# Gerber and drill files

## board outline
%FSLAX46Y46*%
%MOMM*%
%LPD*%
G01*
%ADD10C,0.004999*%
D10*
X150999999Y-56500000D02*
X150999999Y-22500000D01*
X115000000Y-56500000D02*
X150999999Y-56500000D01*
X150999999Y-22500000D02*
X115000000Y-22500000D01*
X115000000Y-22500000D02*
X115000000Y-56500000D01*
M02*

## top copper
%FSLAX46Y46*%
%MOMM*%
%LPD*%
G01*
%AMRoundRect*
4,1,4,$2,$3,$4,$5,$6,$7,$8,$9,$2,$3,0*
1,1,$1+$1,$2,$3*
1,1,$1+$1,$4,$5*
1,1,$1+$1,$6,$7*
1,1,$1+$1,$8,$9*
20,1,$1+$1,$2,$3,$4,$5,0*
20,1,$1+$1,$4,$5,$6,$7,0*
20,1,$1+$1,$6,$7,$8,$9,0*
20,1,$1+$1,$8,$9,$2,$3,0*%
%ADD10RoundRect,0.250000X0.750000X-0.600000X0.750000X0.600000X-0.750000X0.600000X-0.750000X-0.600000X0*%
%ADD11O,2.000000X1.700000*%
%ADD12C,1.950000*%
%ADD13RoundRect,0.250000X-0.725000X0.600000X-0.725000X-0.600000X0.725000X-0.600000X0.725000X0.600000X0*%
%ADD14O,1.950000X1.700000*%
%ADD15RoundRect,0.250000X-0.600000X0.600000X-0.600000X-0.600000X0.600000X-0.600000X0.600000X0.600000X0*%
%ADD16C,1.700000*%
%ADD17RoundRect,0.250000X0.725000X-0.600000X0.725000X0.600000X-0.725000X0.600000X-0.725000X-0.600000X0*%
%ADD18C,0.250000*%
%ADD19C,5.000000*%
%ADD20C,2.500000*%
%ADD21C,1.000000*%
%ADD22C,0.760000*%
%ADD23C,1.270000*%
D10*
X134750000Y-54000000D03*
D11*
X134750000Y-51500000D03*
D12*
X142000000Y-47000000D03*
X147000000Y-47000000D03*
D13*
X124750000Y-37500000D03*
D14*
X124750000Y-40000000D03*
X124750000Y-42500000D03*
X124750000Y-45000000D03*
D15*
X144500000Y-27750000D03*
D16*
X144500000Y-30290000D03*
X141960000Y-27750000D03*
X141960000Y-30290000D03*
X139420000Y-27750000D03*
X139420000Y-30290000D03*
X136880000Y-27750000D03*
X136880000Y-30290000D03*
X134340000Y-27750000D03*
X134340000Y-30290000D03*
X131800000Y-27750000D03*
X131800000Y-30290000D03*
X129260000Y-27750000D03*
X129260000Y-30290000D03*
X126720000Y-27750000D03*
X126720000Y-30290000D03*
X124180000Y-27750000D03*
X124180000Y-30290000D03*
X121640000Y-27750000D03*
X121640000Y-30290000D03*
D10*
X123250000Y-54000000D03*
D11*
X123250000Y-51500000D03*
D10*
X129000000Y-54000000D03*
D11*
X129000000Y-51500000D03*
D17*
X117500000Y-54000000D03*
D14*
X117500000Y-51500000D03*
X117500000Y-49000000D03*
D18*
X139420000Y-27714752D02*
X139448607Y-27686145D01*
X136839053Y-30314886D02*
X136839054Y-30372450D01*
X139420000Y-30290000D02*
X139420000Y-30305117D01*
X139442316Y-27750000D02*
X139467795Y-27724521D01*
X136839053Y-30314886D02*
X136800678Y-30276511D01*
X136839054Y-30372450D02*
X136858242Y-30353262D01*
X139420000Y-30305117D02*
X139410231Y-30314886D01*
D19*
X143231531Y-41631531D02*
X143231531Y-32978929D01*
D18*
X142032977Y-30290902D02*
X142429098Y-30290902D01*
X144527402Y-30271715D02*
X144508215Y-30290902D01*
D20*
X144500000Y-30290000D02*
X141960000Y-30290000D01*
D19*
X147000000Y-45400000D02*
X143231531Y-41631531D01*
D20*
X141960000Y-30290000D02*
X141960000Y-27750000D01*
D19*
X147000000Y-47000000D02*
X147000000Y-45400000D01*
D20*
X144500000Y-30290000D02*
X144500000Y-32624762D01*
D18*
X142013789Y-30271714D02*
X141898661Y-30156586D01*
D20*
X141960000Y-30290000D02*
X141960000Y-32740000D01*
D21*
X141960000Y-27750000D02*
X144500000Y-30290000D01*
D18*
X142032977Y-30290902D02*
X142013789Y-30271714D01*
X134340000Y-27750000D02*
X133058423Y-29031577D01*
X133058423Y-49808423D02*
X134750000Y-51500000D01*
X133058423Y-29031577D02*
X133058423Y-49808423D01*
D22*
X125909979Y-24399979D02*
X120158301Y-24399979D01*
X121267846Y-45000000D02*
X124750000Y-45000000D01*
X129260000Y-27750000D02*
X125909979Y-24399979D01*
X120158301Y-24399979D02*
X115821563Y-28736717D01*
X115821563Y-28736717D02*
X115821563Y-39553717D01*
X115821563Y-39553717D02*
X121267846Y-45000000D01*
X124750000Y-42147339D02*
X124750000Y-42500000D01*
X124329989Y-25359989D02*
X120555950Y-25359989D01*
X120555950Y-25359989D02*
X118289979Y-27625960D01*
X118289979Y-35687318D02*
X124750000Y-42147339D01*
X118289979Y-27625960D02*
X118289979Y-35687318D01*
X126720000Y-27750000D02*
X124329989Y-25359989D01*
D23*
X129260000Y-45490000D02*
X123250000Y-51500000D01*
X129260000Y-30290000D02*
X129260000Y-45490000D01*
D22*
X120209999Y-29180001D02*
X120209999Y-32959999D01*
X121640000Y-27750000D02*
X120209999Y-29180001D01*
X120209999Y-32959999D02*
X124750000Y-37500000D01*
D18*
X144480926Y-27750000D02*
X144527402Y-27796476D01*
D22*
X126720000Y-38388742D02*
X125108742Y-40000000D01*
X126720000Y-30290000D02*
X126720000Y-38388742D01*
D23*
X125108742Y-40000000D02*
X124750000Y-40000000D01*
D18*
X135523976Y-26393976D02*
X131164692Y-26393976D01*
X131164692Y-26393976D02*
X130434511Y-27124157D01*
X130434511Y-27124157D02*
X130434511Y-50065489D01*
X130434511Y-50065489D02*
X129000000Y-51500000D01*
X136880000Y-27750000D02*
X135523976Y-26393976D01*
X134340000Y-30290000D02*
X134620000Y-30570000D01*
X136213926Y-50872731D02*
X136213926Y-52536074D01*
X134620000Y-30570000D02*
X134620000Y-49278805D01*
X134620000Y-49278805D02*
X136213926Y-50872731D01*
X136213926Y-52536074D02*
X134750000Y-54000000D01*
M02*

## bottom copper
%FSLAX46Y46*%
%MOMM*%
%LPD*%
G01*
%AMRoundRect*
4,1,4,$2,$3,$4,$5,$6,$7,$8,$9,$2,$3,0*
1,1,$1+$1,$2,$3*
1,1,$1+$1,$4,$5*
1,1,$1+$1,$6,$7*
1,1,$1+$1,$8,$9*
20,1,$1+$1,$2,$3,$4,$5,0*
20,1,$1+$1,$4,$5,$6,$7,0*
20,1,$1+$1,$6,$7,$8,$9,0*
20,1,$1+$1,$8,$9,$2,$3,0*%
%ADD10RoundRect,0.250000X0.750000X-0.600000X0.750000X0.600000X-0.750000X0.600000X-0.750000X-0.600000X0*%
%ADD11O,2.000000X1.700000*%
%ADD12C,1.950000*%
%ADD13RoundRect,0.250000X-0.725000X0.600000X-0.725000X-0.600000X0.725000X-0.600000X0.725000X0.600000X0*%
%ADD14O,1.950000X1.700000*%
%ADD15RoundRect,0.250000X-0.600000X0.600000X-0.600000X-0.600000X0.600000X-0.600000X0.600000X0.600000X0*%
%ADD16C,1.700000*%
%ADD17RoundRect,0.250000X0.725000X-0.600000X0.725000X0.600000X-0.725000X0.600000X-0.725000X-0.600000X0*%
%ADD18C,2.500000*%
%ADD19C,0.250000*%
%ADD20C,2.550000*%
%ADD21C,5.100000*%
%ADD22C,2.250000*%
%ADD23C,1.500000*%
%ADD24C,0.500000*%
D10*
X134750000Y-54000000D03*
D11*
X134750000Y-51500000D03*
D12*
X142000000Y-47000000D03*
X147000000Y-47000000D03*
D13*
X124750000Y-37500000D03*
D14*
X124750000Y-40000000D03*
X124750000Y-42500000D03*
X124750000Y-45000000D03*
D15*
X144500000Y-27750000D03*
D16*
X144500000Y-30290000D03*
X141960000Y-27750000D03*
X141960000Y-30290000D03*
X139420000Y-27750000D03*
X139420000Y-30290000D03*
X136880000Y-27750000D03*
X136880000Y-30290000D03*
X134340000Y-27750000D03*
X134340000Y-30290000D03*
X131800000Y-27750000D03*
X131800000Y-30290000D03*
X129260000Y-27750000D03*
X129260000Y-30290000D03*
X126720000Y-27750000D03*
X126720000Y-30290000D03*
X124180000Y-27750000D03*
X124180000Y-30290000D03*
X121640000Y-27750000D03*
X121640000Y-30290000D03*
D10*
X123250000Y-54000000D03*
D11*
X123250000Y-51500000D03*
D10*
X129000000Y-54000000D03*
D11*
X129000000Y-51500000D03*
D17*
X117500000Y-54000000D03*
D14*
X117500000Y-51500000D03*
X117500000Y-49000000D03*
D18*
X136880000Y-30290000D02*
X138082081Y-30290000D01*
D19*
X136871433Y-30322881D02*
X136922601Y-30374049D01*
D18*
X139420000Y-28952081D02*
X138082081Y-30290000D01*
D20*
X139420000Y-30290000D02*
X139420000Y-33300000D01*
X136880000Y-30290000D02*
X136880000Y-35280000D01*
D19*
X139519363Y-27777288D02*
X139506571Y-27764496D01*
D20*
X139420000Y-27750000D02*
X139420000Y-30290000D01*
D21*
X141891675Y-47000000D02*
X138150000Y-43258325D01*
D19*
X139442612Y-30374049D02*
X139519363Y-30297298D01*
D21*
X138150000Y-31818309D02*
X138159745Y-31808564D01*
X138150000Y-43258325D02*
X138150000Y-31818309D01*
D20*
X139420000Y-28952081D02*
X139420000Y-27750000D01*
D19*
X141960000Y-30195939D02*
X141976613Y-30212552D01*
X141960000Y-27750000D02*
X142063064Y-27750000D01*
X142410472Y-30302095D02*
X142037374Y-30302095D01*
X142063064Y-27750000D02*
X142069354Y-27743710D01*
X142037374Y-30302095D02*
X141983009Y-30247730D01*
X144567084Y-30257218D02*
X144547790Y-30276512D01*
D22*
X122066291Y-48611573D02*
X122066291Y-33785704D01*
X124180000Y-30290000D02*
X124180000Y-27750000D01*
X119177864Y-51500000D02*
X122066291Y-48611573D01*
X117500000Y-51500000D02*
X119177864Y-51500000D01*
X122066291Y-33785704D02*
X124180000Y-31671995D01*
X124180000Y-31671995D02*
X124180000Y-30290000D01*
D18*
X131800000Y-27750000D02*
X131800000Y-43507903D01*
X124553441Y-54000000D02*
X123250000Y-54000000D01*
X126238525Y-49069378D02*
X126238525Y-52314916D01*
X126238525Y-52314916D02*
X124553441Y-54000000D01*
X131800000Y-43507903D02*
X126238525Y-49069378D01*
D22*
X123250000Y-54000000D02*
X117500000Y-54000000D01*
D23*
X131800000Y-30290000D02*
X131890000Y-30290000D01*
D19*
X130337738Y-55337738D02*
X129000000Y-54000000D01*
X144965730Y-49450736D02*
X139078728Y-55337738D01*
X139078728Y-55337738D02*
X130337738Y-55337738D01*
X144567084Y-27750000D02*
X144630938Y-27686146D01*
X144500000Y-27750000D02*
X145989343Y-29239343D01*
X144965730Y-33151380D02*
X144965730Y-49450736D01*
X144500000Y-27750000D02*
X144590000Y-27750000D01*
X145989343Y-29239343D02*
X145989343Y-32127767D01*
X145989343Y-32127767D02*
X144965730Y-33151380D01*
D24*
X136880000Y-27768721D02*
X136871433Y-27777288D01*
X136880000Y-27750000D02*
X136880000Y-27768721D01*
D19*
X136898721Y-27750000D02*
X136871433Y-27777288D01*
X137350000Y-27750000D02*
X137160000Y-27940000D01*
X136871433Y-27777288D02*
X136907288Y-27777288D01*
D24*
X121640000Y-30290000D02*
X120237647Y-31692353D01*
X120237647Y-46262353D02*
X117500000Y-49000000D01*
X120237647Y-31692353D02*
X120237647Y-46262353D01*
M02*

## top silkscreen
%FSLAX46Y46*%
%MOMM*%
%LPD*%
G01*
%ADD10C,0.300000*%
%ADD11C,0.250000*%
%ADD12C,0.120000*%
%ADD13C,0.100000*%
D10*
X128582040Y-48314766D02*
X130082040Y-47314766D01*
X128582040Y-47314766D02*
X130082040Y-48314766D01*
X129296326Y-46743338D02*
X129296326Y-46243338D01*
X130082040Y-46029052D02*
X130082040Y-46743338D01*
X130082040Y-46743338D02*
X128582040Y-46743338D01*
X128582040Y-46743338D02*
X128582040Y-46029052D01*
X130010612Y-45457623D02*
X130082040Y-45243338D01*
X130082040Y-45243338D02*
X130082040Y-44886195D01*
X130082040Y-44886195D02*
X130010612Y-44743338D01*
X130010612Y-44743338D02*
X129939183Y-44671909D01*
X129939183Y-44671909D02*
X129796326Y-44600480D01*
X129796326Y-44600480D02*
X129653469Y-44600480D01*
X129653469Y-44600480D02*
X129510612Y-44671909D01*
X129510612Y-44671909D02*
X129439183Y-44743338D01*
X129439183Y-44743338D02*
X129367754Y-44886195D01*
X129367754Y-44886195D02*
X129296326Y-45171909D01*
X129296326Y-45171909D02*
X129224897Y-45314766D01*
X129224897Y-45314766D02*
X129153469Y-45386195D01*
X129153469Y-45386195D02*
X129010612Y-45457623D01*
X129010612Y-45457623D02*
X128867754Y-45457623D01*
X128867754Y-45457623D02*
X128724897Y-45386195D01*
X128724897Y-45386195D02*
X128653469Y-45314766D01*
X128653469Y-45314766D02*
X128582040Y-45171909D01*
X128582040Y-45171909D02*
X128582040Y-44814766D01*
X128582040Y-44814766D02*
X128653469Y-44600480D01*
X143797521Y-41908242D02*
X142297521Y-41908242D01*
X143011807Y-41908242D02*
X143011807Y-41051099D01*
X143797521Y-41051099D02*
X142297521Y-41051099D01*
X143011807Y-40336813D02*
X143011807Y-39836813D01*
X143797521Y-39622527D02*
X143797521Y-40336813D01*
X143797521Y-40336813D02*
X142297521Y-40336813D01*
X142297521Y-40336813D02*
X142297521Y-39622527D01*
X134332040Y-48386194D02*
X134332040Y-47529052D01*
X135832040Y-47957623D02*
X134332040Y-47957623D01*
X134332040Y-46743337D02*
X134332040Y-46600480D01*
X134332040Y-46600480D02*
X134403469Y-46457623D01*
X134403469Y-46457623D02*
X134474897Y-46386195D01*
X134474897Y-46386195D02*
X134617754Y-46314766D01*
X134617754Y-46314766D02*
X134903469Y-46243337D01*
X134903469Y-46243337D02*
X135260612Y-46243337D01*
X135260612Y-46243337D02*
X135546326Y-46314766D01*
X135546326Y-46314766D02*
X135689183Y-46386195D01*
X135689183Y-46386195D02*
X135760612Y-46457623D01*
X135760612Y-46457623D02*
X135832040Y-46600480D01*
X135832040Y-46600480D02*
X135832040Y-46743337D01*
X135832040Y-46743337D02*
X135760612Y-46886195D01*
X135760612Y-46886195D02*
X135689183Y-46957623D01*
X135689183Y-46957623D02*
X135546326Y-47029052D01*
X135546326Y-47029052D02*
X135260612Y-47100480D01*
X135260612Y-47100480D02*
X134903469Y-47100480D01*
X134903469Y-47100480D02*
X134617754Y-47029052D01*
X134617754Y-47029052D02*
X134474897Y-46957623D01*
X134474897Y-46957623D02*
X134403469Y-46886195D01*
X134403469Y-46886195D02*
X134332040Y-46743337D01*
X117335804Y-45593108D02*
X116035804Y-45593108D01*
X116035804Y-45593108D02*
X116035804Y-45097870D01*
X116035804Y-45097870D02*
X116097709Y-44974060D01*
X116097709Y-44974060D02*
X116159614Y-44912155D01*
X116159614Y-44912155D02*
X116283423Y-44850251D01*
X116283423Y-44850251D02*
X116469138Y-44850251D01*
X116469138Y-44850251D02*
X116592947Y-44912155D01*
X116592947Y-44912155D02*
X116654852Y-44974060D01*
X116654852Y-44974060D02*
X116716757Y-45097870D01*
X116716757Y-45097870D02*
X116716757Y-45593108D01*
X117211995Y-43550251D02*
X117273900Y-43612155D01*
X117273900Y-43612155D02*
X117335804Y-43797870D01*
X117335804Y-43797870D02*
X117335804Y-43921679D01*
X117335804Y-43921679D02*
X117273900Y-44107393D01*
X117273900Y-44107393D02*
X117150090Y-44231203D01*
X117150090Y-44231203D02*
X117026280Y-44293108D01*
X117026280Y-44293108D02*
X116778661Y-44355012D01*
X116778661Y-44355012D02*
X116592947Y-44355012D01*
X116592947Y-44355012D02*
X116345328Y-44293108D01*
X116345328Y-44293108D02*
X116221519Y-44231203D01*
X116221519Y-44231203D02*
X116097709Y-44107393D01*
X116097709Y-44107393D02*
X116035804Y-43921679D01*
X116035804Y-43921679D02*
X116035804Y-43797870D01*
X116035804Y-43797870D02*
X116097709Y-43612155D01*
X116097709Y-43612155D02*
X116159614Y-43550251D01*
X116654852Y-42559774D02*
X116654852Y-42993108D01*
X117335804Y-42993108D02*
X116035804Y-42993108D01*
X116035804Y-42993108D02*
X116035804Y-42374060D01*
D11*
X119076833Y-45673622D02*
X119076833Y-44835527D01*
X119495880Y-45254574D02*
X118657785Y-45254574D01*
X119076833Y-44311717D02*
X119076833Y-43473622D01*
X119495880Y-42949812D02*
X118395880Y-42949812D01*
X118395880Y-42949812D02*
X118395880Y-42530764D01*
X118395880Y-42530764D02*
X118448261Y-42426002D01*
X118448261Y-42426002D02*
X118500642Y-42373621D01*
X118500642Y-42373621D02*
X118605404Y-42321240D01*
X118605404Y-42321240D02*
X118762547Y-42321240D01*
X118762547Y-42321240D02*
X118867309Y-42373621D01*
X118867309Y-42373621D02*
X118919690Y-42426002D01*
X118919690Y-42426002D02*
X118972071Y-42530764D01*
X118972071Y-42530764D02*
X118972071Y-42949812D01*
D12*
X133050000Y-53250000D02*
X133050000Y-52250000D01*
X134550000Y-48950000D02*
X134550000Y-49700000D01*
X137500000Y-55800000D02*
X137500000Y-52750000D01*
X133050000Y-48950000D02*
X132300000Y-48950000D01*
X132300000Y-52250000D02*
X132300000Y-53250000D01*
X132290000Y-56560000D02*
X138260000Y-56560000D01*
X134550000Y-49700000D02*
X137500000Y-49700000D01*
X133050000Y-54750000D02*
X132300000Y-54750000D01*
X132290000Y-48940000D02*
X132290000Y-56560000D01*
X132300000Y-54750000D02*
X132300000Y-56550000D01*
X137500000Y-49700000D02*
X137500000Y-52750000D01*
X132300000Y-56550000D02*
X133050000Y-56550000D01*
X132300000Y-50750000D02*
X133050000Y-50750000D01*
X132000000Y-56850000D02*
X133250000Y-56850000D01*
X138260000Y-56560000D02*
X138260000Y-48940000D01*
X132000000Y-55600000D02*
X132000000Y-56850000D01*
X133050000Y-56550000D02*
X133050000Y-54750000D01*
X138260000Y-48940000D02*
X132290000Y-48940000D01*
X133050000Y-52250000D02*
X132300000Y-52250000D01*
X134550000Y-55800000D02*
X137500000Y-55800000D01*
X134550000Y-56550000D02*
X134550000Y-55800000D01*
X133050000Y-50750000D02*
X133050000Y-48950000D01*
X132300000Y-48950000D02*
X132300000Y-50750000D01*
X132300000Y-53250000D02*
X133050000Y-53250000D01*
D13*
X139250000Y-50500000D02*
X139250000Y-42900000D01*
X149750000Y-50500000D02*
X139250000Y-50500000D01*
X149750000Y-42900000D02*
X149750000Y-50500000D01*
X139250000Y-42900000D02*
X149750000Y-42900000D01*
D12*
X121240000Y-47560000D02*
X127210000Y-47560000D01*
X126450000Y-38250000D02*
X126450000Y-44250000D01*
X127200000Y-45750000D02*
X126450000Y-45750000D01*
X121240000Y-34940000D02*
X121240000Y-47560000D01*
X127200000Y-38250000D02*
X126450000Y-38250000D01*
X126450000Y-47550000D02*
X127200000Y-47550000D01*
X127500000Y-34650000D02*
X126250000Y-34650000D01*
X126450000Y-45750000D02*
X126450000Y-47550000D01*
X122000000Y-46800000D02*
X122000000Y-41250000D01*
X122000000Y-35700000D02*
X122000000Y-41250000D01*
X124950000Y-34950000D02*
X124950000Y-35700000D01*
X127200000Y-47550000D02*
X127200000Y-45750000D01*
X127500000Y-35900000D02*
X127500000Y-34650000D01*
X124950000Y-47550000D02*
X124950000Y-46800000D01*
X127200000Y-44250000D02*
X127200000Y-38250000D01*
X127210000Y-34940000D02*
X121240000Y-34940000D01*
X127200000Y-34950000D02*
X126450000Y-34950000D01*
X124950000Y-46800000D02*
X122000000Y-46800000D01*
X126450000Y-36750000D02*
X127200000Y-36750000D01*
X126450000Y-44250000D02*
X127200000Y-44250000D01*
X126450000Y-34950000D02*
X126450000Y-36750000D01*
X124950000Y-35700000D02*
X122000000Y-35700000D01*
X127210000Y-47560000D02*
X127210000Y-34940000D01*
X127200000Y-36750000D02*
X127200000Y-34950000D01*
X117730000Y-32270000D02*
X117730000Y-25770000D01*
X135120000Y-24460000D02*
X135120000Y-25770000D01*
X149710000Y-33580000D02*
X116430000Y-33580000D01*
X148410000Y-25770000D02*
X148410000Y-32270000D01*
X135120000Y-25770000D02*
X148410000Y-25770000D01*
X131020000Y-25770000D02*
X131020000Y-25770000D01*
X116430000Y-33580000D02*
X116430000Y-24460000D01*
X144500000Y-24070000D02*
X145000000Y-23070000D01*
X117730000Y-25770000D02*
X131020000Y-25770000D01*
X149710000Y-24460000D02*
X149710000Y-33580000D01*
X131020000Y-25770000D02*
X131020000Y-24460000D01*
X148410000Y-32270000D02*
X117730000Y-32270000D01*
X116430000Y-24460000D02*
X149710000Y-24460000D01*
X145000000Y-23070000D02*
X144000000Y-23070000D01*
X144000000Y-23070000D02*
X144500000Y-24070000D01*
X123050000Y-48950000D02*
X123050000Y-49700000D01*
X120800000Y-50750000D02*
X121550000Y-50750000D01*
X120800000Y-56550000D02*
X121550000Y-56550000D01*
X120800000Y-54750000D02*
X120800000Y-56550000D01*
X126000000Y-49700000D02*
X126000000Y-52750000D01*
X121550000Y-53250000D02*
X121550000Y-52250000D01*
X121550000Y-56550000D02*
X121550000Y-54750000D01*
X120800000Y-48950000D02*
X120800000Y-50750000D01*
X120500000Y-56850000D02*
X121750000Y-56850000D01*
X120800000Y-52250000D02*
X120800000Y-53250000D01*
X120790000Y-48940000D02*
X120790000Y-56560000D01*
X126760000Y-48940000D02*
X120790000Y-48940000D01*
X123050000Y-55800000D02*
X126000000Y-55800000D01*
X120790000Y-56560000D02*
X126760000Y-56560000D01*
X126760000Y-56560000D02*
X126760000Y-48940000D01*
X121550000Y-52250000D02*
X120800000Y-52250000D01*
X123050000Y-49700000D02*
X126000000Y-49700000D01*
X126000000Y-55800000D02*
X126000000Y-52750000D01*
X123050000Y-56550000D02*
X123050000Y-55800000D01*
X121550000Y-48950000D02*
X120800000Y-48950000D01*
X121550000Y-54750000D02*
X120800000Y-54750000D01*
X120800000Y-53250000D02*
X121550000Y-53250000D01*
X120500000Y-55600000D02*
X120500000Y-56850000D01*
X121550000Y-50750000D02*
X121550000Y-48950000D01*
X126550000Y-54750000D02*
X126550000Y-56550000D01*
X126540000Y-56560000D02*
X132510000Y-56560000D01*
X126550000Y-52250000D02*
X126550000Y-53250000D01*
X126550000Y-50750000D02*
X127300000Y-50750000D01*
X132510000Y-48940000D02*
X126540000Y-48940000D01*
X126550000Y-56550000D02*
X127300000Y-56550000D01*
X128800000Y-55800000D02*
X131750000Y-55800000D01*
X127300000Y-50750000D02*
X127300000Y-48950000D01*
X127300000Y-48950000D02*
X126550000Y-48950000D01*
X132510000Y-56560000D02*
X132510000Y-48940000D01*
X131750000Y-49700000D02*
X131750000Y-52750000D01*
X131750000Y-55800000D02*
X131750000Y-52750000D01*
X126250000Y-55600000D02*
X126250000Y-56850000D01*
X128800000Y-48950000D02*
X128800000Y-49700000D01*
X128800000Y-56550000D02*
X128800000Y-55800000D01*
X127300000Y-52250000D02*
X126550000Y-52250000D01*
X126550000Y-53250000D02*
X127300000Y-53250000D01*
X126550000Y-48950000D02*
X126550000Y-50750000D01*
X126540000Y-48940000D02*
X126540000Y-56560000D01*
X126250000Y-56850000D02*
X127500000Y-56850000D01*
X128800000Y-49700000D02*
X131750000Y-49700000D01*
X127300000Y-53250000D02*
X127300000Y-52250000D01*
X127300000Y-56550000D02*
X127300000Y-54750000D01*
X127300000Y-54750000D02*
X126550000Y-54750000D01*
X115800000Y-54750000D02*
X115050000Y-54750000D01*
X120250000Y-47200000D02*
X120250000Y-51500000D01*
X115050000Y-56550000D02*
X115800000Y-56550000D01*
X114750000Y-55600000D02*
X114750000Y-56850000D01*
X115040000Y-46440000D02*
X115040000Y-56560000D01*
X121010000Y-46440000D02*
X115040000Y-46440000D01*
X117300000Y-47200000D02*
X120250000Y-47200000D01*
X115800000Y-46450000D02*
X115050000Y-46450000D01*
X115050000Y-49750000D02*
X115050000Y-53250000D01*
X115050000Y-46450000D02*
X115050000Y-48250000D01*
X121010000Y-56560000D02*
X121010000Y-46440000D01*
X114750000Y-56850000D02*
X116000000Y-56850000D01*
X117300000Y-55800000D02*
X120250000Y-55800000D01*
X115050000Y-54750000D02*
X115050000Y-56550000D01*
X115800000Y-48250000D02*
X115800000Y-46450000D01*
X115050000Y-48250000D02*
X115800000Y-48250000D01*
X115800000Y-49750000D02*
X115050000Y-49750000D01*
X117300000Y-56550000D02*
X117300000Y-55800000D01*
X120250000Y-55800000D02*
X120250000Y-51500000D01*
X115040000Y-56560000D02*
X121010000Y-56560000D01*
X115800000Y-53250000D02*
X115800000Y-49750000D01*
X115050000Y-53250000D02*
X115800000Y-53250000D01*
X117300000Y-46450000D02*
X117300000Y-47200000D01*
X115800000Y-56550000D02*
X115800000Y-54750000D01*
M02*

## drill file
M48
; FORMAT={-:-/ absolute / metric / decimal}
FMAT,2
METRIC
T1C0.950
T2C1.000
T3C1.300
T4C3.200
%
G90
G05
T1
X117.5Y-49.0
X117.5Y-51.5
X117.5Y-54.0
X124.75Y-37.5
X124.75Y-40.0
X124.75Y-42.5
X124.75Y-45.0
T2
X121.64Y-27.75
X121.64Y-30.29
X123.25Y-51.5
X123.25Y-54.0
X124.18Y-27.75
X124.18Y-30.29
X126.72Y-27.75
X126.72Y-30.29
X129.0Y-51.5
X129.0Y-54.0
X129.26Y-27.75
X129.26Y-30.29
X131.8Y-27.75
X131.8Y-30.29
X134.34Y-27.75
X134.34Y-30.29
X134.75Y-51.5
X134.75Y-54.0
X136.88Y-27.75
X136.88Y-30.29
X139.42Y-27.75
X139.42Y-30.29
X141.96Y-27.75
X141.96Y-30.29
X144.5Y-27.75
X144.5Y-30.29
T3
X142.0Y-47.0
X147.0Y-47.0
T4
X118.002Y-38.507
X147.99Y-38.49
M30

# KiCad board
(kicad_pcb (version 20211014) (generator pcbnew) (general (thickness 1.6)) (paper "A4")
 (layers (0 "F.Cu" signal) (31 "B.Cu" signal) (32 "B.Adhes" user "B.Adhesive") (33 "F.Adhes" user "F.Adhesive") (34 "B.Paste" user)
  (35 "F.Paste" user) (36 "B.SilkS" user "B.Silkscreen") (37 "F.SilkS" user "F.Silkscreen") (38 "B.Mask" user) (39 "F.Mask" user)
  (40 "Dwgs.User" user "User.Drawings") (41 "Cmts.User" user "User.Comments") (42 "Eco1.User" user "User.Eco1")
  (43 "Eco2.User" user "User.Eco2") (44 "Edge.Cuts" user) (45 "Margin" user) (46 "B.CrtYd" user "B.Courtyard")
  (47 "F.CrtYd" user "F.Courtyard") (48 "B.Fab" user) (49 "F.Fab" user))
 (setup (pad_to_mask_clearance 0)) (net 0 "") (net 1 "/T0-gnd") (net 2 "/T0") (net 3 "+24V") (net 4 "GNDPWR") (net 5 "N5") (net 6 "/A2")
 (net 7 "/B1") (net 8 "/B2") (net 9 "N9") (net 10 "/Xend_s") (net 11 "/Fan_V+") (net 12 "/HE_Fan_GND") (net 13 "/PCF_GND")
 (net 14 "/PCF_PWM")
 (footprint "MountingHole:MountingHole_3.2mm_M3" (layer "F.Cu") (at 118.001564 38.507316)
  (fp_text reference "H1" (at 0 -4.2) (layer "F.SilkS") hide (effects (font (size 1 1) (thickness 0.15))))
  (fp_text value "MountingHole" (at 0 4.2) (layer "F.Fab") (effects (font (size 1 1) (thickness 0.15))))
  (pad "" np_thru_hole circle locked (at 0 0) (size 3.2 3.2) (drill 3.2) (layers *.Cu *.Mask)))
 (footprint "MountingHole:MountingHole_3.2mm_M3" (layer "F.Cu") (at 147.990137 38.490139)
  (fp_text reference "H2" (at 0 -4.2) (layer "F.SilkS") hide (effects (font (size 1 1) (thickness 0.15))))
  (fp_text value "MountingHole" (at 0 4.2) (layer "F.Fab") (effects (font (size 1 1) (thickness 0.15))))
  (pad "" np_thru_hole circle locked (at 0 0) (size 3.2 3.2) (drill 3.2) (layers *.Cu *.Mask)))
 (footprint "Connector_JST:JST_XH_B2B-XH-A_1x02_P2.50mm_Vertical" (layer "F.Cu") (at 134.75 54 90)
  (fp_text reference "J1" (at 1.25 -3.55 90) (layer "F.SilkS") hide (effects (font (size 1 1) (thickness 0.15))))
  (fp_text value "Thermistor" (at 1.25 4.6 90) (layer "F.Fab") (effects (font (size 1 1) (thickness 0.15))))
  (fp_line (start 0.75 -1.7) (end 1.75 -1.7) (layer "F.SilkS") (width 0.12))
  (fp_line (start 5.05 -0.2) (end 4.3 -0.2) (layer "F.SilkS") (width 0.12))
  (fp_line (start -1.8 2.75) (end 1.25 2.75) (layer "F.SilkS") (width 0.12))
  (fp_line (start 5.05 -1.7) (end 5.05 -2.45) (layer "F.SilkS") (width 0.12))
  (fp_line (start 1.75 -2.45) (end 0.75 -2.45) (layer "F.SilkS") (width 0.12))
  (fp_line (start -2.56 -2.46) (end -2.56 3.51) (layer "F.SilkS") (width 0.12))
  (fp_line (start 4.3 -0.2) (end 4.3 2.75) (layer "F.SilkS") (width 0.12))
  (fp_line (start -0.75 -1.7) (end -0.75 -2.45) (layer "F.SilkS") (width 0.12))
  (fp_line (start 5.06 -2.46) (end -2.56 -2.46) (layer "F.SilkS") (width 0.12))
  (fp_line (start -0.75 -2.45) (end -2.55 -2.45) (layer "F.SilkS") (width 0.12))
  (fp_line (start 4.3 2.75) (end 1.25 2.75) (layer "F.SilkS") (width 0.12))
  (fp_line (start -2.55 -2.45) (end -2.55 -1.7) (layer "F.SilkS") (width 0.12))
  (fp_line (start 3.25 -2.45) (end 3.25 -1.7) (layer "F.SilkS") (width 0.12))
  (fp_line (start -2.85 -2.75) (end -2.85 -1.5) (layer "F.SilkS") (width 0.12))
  (fp_line (start -2.56 3.51) (end 5.06 3.51) (layer "F.SilkS") (width 0.12))
  (fp_line (start -1.6 -2.75) (end -2.85 -2.75) (layer "F.SilkS") (width 0.12))
  (fp_line (start -2.55 -1.7) (end -0.75 -1.7) (layer "F.SilkS") (width 0.12))
  (fp_line (start 5.06 3.51) (end 5.06 -2.46) (layer "F.SilkS") (width 0.12))
  (fp_line (start 1.75 -1.7) (end 1.75 -2.45) (layer "F.SilkS") (width 0.12))
  (fp_line (start -1.8 -0.2) (end -1.8 2.75) (layer "F.SilkS") (width 0.12))
  (fp_line (start -2.55 -0.2) (end -1.8 -0.2) (layer "F.SilkS") (width 0.12))
  (fp_line (start 3.25 -1.7) (end 5.05 -1.7) (layer "F.SilkS") (width 0.12))
  (fp_line (start 5.05 -2.45) (end 3.25 -2.45) (layer "F.SilkS") (width 0.12))
  (fp_line (start 0.75 -2.45) (end 0.75 -1.7) (layer "F.SilkS") (width 0.12))
  (pad "1" thru_hole roundrect locked (at 0 0 90) (size 1.7 2) (drill 1) (layers *.Cu *.Mask) (roundrect_rratio 0.1470588235)
   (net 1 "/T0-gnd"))
  (pad "2" thru_hole oval locked (at 2.5 0 90) (size 1.7 2) (drill 1) (layers *.Cu *.Mask) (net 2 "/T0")))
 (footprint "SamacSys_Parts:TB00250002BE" (layer "F.Cu") (at 142 47)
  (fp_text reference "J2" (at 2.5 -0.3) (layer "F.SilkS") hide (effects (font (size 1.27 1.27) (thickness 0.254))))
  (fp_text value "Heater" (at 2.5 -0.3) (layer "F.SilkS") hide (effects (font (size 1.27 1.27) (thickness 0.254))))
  (fp_line (start -2.75 3.5) (end -2.75 -4.1) (layer "F.SilkS") (width 0.1))
  (fp_line (start 7.75 3.5) (end -2.75 3.5) (layer "F.SilkS") (width 0.1))
  (fp_line (start 7.75 -4.1) (end 7.75 3.5) (layer "F.SilkS") (width 0.1))
  (fp_line (start -2.75 -4.1) (end 7.75 -4.1) (layer "F.SilkS") (width 0.1))
  (pad "1" thru_hole circle locked (at 0 0) (size 1.95 1.95) (drill 1.3) (layers *.Cu *.Mask) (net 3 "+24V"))
  (pad "2" thru_hole circle locked (at 5 0) (size 1.95 1.95) (drill 1.3) (layers *.Cu *.Mask) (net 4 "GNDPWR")))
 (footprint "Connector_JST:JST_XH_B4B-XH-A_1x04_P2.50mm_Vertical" (layer "F.Cu") (at 124.75 37.5 -90)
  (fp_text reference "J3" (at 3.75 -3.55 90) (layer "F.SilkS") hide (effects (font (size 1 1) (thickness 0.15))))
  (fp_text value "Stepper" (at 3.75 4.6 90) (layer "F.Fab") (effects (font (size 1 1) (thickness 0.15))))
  (fp_line (start 10.06 3.51) (end 10.06 -2.46) (layer "F.SilkS") (width 0.12))
  (fp_line (start 0.75 -1.7) (end 6.75 -1.7) (layer "F.SilkS") (width 0.12))
  (fp_line (start 8.25 -2.45) (end 8.25 -1.7) (layer "F.SilkS") (width 0.12))
  (fp_line (start -2.56 3.51) (end 10.06 3.51) (layer "F.SilkS") (width 0.12))
  (fp_line (start 0.75 -2.45) (end 0.75 -1.7) (layer "F.SilkS") (width 0.12))
  (fp_line (start 10.05 -1.7) (end 10.05 -2.45) (layer "F.SilkS") (width 0.12))
  (fp_line (start -2.85 -2.75) (end -2.85 -1.5) (layer "F.SilkS") (width 0.12))
  (fp_line (start 8.25 -1.7) (end 10.05 -1.7) (layer "F.SilkS") (width 0.12))
  (fp_line (start 9.3 2.75) (end 3.75 2.75) (layer "F.SilkS") (width 0.12))
  (fp_line (start -1.8 2.75) (end 3.75 2.75) (layer "F.SilkS") (width 0.12))
  (fp_line (start -2.55 -0.2) (end -1.8 -0.2) (layer "F.SilkS") (width 0.12))
  (fp_line (start 10.05 -2.45) (end 8.25 -2.45) (layer "F.SilkS") (width 0.12))
  (fp_line (start -1.6 -2.75) (end -2.85 -2.75) (layer "F.SilkS") (width 0.12))
  (fp_line (start 10.05 -0.2) (end 9.3 -0.2) (layer "F.SilkS") (width 0.12))
  (fp_line (start 6.75 -2.45) (end 0.75 -2.45) (layer "F.SilkS") (width 0.12))
  (fp_line (start -2.56 -2.46) (end -2.56 3.51) (layer "F.SilkS") (width 0.12))
  (fp_line (start -2.55 -2.45) (end -2.55 -1.7) (layer "F.SilkS") (width 0.12))
  (fp_line (start 9.3 -0.2) (end 9.3 2.75) (layer "F.SilkS") (width 0.12))
  (fp_line (start -0.75 -1.7) (end -0.75 -2.45) (layer "F.SilkS") (width 0.12))
  (fp_line (start 6.75 -1.7) (end 6.75 -2.45) (layer "F.SilkS") (width 0.12))
  (fp_line (start -2.55 -1.7) (end -0.75 -1.7) (layer "F.SilkS") (width 0.12))
  (fp_line (start -1.8 -0.2) (end -1.8 2.75) (layer "F.SilkS") (width 0.12))
  (fp_line (start 10.06 -2.46) (end -2.56 -2.46) (layer "F.SilkS") (width 0.12))
  (fp_line (start -0.75 -2.45) (end -2.55 -2.45) (layer "F.SilkS") (width 0.12))
  (pad "1" thru_hole roundrect locked (at 0 0 270) (size 1.7 1.95) (drill 0.95) (layers *.Cu *.Mask) (roundrect_rratio 0.1470588235)
   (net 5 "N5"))
  (pad "2" thru_hole oval locked (at 2.5 0 270) (size 1.7 1.95) (drill 0.95) (layers *.Cu *.Mask) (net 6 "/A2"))
  (pad "3" thru_hole oval locked (at 5 0 270) (size 1.7 1.95) (drill 0.95) (layers *.Cu *.Mask) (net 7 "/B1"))
  (pad "4" thru_hole oval locked (at 7.5 0 270) (size 1.7 1.95) (drill 0.95) (layers *.Cu *.Mask) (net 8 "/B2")))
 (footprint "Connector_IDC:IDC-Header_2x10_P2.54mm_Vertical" (layer "F.Cu") (at 144.5 27.75 -90)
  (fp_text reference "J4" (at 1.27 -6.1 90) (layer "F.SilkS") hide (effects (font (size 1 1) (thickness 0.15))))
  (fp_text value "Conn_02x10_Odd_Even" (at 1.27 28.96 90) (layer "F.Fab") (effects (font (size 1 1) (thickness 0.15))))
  (fp_line (start 4.52 26.77) (end -1.98 26.77) (layer "F.SilkS") (width 0.12))
  (fp_line (start -3.29 9.38) (end -1.98 9.38) (layer "F.SilkS") (width 0.12))
  (fp_line (start 5.83 -5.21) (end 5.83 28.07) (layer "F.SilkS") (width 0.12))
  (fp_line (start -1.98 -3.91) (end 4.52 -3.91) (layer "F.SilkS") (width 0.12))
  (fp_line (start -1.98 9.38) (end -1.98 -3.91) (layer "F.SilkS") (width 0.12))
  (fp_line (start -1.98 13.48) (end -1.98 13.48) (layer "F.SilkS") (width 0.12))
  (fp_line (start 5.83 28.07) (end -3.29 28.07) (layer "F.SilkS") (width 0.12))
  (fp_line (start -3.68 0) (end -4.68 -0.5) (layer "F.SilkS") (width 0.12))
  (fp_line (start -1.98 26.77) (end -1.98 13.48) (layer "F.SilkS") (width 0.12))
  (fp_line (start -3.29 -5.21) (end 5.83 -5.21) (layer "F.SilkS") (width 0.12))
  (fp_line (start -1.98 13.48) (end -3.29 13.48) (layer "F.SilkS") (width 0.12))
  (fp_line (start 4.52 -3.91) (end 4.52 26.77) (layer "F.SilkS") (width 0.12))
  (fp_line (start -3.29 28.07) (end -3.29 -5.21) (layer "F.SilkS") (width 0.12))
  (fp_line (start -4.68 -0.5) (end -4.68 0.5) (layer "F.SilkS") (width 0.12))
  (fp_line (start -4.68 0.5) (end -3.68 0) (layer "F.SilkS") (width 0.12))
  (pad "1" thru_hole roundrect locked (at 0 0 270) (size 1.7 1.7) (drill 1) (layers *.Cu *.Mask) (roundrect_rratio 0.1470588235)
   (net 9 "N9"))
  (pad "2" thru_hole circle locked (at 2.54 0 270) (size 1.7 1.7) (drill 1) (layers *.Cu *.Mask) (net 4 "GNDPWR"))
  (pad "3" thru_hole circle locked (at 0 2.54 270) (size 1.7 1.7) (drill 1) (layers *.Cu *.Mask) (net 4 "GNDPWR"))
  (pad "4" thru_hole circle locked (at 2.54 2.54 270) (size 1.7 1.7) (drill 1) (layers *.Cu *.Mask) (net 4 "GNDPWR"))
  (pad "5" thru_hole circle locked (at 0 5.08 270) (size 1.7 1.7) (drill 1) (layers *.Cu *.Mask) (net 3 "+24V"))
  (pad "6" thru_hole circle locked (at 2.54 5.08 270) (size 1.7 1.7) (drill 1) (layers *.Cu *.Mask) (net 3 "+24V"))
  (pad "7" thru_hole circle locked (at 0 7.62 270) (size 1.7 1.7) (drill 1) (layers *.Cu *.Mask) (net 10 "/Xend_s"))
  (pad "8" thru_hole circle locked (at 2.54 7.62 270) (size 1.7 1.7) (drill 1) (layers *.Cu *.Mask) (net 3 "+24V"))
  (pad "9" thru_hole circle locked (at 0 10.16 270) (size 1.7 1.7) (drill 1) (layers *.Cu *.Mask) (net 2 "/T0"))
  (pad "10" thru_hole circle locked (at 2.54 10.16 270) (size 1.7 1.7) (drill 1) (layers *.Cu *.Mask) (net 1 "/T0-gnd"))
  (pad "11" thru_hole circle locked (at 0 12.7 270) (size 1.7 1.7) (drill 1) (layers *.Cu *.Mask) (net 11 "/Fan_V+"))
  (pad "12" thru_hole circle locked (at 2.54 12.7 270) (size 1.7 1.7) (drill 1) (layers *.Cu *.Mask) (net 11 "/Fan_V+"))
  (pad "13" thru_hole circle locked (at 0 15.24 270) (size 1.7 1.7) (drill 1) (layers *.Cu *.Mask) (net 8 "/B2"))
  (pad "14" thru_hole circle locked (at 2.54 15.24 270) (size 1.7 1.7) (drill 1) (layers *.Cu *.Mask) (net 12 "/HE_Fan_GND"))
  (pad "15" thru_hole circle locked (at 0 17.78 270) (size 1.7 1.7) (drill 1) (layers *.Cu *.Mask) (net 7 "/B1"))
  (pad "16" thru_hole circle locked (at 2.54 17.78 270) (size 1.7 1.7) (drill 1) (layers *.Cu *.Mask) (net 6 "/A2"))
  (pad "17" thru_hole circle locked (at 0 20.32 270) (size 1.7 1.7) (drill 1) (layers *.Cu *.Mask) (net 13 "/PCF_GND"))
  (pad "18" thru_hole circle locked (at 2.54 20.32 270) (size 1.7 1.7) (drill 1) (layers *.Cu *.Mask) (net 13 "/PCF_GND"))
  (pad "19" thru_hole circle locked (at 0 22.86 270) (size 1.7 1.7) (drill 1) (layers *.Cu *.Mask) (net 5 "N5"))
  (pad "20" thru_hole circle locked (at 2.54 22.86 270) (size 1.7 1.7) (drill 1) (layers *.Cu *.Mask) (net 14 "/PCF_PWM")))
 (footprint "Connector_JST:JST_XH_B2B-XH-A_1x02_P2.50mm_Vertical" (layer "F.Cu") (at 123.25 54 90)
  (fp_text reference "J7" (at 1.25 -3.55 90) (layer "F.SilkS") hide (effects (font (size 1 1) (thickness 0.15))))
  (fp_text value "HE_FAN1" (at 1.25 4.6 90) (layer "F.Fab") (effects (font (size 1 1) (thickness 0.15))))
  (fp_line (start 5.05 -0.2) (end 4.3 -0.2) (layer "F.SilkS") (width 0.12))
  (fp_line (start 3.25 -2.45) (end 3.25 -1.7) (layer "F.SilkS") (width 0.12))
  (fp_line (start -2.55 -2.45) (end -2.55 -1.7) (layer "F.SilkS") (width 0.12))
  (fp_line (start -0.75 -2.45) (end -2.55 -2.45) (layer "F.SilkS") (width 0.12))
  (fp_line (start 4.3 2.75) (end 1.25 2.75) (layer "F.SilkS") (width 0.12))
  (fp_line (start 0.75 -1.7) (end 1.75 -1.7) (layer "F.SilkS") (width 0.12))
  (fp_line (start -2.55 -1.7) (end -0.75 -1.7) (layer "F.SilkS") (width 0.12))
  (fp_line (start 5.05 -2.45) (end 3.25 -2.45) (layer "F.SilkS") (width 0.12))
  (fp_line (start -2.85 -2.75) (end -2.85 -1.5) (layer "F.SilkS") (width 0.12))
  (fp_line (start 1.75 -2.45) (end 0.75 -2.45) (layer "F.SilkS") (width 0.12))
  (fp_line (start 5.06 -2.46) (end -2.56 -2.46) (layer "F.SilkS") (width 0.12))
  (fp_line (start 5.06 3.51) (end 5.06 -2.46) (layer "F.SilkS") (width 0.12))
  (fp_line (start -1.8 -0.2) (end -1.8 2.75) (layer "F.SilkS") (width 0.12))
  (fp_line (start -2.56 -2.46) (end -2.56 3.51) (layer "F.SilkS") (width 0.12))
  (fp_line (start -2.56 3.51) (end 5.06 3.51) (layer "F.SilkS") (width 0.12))
  (fp_line (start 1.75 -1.7) (end 1.75 -2.45) (layer "F.SilkS") (width 0.12))
  (fp_line (start 4.3 -0.2) (end 4.3 2.75) (layer "F.SilkS") (width 0.12))
  (fp_line (start -1.8 2.75) (end 1.25 2.75) (layer "F.SilkS") (width 0.12))
  (fp_line (start -2.55 -0.2) (end -1.8 -0.2) (layer "F.SilkS") (width 0.12))
  (fp_line (start 5.05 -1.7) (end 5.05 -2.45) (layer "F.SilkS") (width 0.12))
  (fp_line (start -0.75 -1.7) (end -0.75 -2.45) (layer "F.SilkS") (width 0.12))
  (fp_line (start 0.75 -2.45) (end 0.75 -1.7) (layer "F.SilkS") (width 0.12))
  (fp_line (start -1.6 -2.75) (end -2.85 -2.75) (layer "F.SilkS") (width 0.12))
  (fp_line (start 3.25 -1.7) (end 5.05 -1.7) (layer "F.SilkS") (width 0.12))
  (pad "1" thru_hole roundrect locked (at 0 0 90) (size 1.7 2) (drill 1) (layers *.Cu *.Mask) (roundrect_rratio 0.1470588235)
   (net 11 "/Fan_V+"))
  (pad "2" thru_hole oval locked (at 2.5 0 90) (size 1.7 2) (drill 1) (layers *.Cu *.Mask) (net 12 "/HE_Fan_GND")))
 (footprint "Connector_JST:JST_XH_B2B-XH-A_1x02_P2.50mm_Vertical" (layer "F.Cu") (at 129 54 90)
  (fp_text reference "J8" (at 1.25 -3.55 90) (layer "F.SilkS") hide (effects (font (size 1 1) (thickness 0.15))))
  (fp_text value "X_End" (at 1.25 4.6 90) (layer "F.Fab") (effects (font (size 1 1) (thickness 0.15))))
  (fp_line (start -0.75 -2.45) (end -2.55 -2.45) (layer "F.SilkS") (width 0.12))
  (fp_line (start -2.56 -2.46) (end -2.56 3.51) (layer "F.SilkS") (width 0.12))
  (fp_line (start 1.75 -2.45) (end 0.75 -2.45) (layer "F.SilkS") (width 0.12))
  (fp_line (start 3.25 -2.45) (end 3.25 -1.7) (layer "F.SilkS") (width 0.12))
  (fp_line (start 5.06 3.51) (end 5.06 -2.46) (layer "F.SilkS") (width 0.12))
  (fp_line (start -2.55 -2.45) (end -2.55 -1.7) (layer "F.SilkS") (width 0.12))
  (fp_line (start -1.8 -0.2) (end -1.8 2.75) (layer "F.SilkS") (width 0.12))
  (fp_line (start 3.25 -1.7) (end 5.05 -1.7) (layer "F.SilkS") (width 0.12))
  (fp_line (start 5.05 -1.7) (end 5.05 -2.45) (layer "F.SilkS") (width 0.12))
  (fp_line (start -2.56 3.51) (end 5.06 3.51) (layer "F.SilkS") (width 0.12))
  (fp_line (start 4.3 2.75) (end 1.25 2.75) (layer "F.SilkS") (width 0.12))
  (fp_line (start -1.8 2.75) (end 1.25 2.75) (layer "F.SilkS") (width 0.12))
  (fp_line (start -1.6 -2.75) (end -2.85 -2.75) (layer "F.SilkS") (width 0.12))
  (fp_line (start 5.05 -0.2) (end 4.3 -0.2) (layer "F.SilkS") (width 0.12))
  (fp_line (start -2.55 -0.2) (end -1.8 -0.2) (layer "F.SilkS") (width 0.12))
  (fp_line (start 1.75 -1.7) (end 1.75 -2.45) (layer "F.SilkS") (width 0.12))
  (fp_line (start 0.75 -2.45) (end 0.75 -1.7) (layer "F.SilkS") (width 0.12))
  (fp_line (start 5.05 -2.45) (end 3.25 -2.45) (layer "F.SilkS") (width 0.12))
  (fp_line (start 5.06 -2.46) (end -2.56 -2.46) (layer "F.SilkS") (width 0.12))
  (fp_line (start -2.85 -2.75) (end -2.85 -1.5) (layer "F.SilkS") (width 0.12))
  (fp_line (start 4.3 -0.2) (end 4.3 2.75) (layer "F.SilkS") (width 0.12))
  (fp_line (start 0.75 -1.7) (end 1.75 -1.7) (layer "F.SilkS") (width 0.12))
  (fp_line (start -2.55 -1.7) (end -0.75 -1.7) (layer "F.SilkS") (width 0.12))
  (fp_line (start -0.75 -1.7) (end -0.75 -2.45) (layer "F.SilkS") (width 0.12))
  (pad "1" thru_hole roundrect locked (at 0 0 90) (size 1.7 2) (drill 1) (layers *.Cu *.Mask) (roundrect_rratio 0.1470588235) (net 9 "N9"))
  (pad "2" thru_hole oval locked (at 2.5 0 90) (size 1.7 2) (drill 1) (layers *.Cu *.Mask) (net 10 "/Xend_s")))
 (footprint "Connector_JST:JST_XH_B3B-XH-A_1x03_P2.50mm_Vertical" (layer "F.Cu") (at 117.5 54 90)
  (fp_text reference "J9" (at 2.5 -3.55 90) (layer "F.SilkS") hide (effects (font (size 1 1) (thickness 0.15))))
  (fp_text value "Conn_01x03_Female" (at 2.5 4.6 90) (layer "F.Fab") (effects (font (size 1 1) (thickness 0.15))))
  (fp_line (start -0.75 -1.7) (end -0.75 -2.45) (layer "F.SilkS") (width 0.12))
  (fp_line (start 6.8 2.75) (end 2.5 2.75) (layer "F.SilkS") (width 0.12))
  (fp_line (start -2.55 -2.45) (end -2.55 -1.7) (layer "F.SilkS") (width 0.12))
  (fp_line (start -1.6 -2.75) (end -2.85 -2.75) (layer "F.SilkS") (width 0.12))
  (fp_line (start 7.56 -2.46) (end -2.56 -2.46) (layer "F.SilkS") (width 0.12))
  (fp_line (start 7.56 3.51) (end 7.56 -2.46) (layer "F.SilkS") (width 0.12))
  (fp_line (start 6.8 -0.2) (end 6.8 2.75) (layer "F.SilkS") (width 0.12))
  (fp_line (start 7.55 -1.7) (end 7.55 -2.45) (layer "F.SilkS") (width 0.12))
  (fp_line (start 4.25 -2.45) (end 0.75 -2.45) (layer "F.SilkS") (width 0.12))
  (fp_line (start 7.55 -2.45) (end 5.75 -2.45) (layer "F.SilkS") (width 0.12))
  (fp_line (start -2.56 3.51) (end 7.56 3.51) (layer "F.SilkS") (width 0.12))
  (fp_line (start -2.85 -2.75) (end -2.85 -1.5) (layer "F.SilkS") (width 0.12))
  (fp_line (start -1.8 -0.2) (end -1.8 2.75) (layer "F.SilkS") (width 0.12))
  (fp_line (start -0.75 -2.45) (end -2.55 -2.45) (layer "F.SilkS") (width 0.12))
  (fp_line (start 5.75 -1.7) (end 7.55 -1.7) (layer "F.SilkS") (width 0.12))
  (fp_line (start 5.75 -2.45) (end 5.75 -1.7) (layer "F.SilkS") (width 0.12))
  (fp_line (start 4.25 -1.7) (end 4.25 -2.45) (layer "F.SilkS") (width 0.12))
  (fp_line (start -2.55 -0.2) (end -1.8 -0.2) (layer "F.SilkS") (width 0.12))
  (fp_line (start -1.8 2.75) (end 2.5 2.75) (layer "F.SilkS") (width 0.12))
  (fp_line (start -2.56 -2.46) (end -2.56 3.51) (layer "F.SilkS") (width 0.12))
  (fp_line (start 0.75 -1.7) (end 4.25 -1.7) (layer "F.SilkS") (width 0.12))
  (fp_line (start 0.75 -2.45) (end 0.75 -1.7) (layer "F.SilkS") (width 0.12))
  (fp_line (start 7.55 -0.2) (end 6.8 -0.2) (layer "F.SilkS") (width 0.12))
  (fp_line (start -2.55 -1.7) (end -0.75 -1.7) (layer "F.SilkS") (width 0.12))
  (pad "1" thru_hole roundrect (at 0 0 90) (size 1.7 1.95) (drill 0.95) (layers *.Cu *.Mask) (roundrect_rratio 0.1470588235)
   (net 11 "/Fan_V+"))
  (pad "2" thru_hole oval (at 2.5 0 90) (size 1.7 1.95) (drill 0.95) (layers *.Cu *.Mask) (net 13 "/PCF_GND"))
  (pad "3" thru_hole oval (at 5 0 90) (size 1.7 1.95) (drill 0.95) (layers *.Cu *.Mask) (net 14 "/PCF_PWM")))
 (gr_line (start 150.999999 56.5) (end 150.999999 22.5) (layer "Edge.Cuts") (width 0.004999))
 (gr_line (start 115 56.5) (end 150.999999 56.5) (layer "Edge.Cuts") (width 0.004999))
 (gr_line (start 150.999999 22.5) (end 115 22.5) (layer "Edge.Cuts") (width 0.004999))
 (gr_line (start 115 22.5) (end 115 56.5) (layer "Edge.Cuts") (width 0.004999))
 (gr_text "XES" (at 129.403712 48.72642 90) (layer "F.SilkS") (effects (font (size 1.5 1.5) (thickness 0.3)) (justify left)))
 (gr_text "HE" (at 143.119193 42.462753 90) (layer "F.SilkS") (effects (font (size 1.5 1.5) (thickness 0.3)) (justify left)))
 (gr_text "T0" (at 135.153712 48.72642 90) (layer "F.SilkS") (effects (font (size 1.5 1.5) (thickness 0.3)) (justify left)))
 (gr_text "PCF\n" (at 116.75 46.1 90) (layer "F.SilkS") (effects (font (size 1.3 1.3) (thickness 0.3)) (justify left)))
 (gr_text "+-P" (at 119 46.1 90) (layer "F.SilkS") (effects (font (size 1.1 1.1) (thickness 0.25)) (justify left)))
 (segment (start 139.42 27.714752) (end 139.448607 27.686145) (width 0.25) (layer "F.Cu") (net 3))
 (segment (start 136.839053 30.314886) (end 136.839054 30.37245) (width 0.25) (layer "F.Cu") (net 3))
 (segment (start 139.42 30.29) (end 139.42 30.305117) (width 0.25) (layer "F.Cu") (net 3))
 (segment (start 139.442316 27.75) (end 139.467795 27.724521) (width 0.25) (layer "F.Cu") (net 3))
 (segment (start 136.839053 30.314886) (end 136.800678 30.276511) (width 0.25) (layer "F.Cu") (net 3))
 (segment (start 136.839054 30.37245) (end 136.858242 30.353262) (width 0.25) (layer "F.Cu") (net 3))
 (segment (start 139.42 30.305117) (end 139.410231 30.314886) (width 0.25) (layer "F.Cu") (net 3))
 (segment (start 136.88 30.29) (end 138.082081 30.29) (width 2.5) (layer "B.Cu") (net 3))
 (segment (start 136.871433 30.322881) (end 136.922601 30.374049) (width 0.25) (layer "B.Cu") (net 3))
 (segment (start 139.42 28.952081) (end 138.082081 30.29) (width 2.5) (layer "B.Cu") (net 3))
 (segment (start 139.42 30.29) (end 139.42 33.3) (width 2.55) (layer "B.Cu") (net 3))
 (segment (start 136.88 30.29) (end 136.88 35.28) (width 2.55) (layer "B.Cu") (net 3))
 (segment (start 139.519363 27.777288) (end 139.506571 27.764496) (width 0.25) (layer "B.Cu") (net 3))
 (segment (start 139.42 27.75) (end 139.42 30.29) (width 2.55) (layer "B.Cu") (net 3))
 (segment (start 141.891675 47) (end 138.15 43.258325) (width 5.1) (layer "B.Cu") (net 3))
 (segment (start 139.442612 30.374049) (end 139.519363 30.297298) (width 0.25) (layer "B.Cu") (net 3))
 (segment (start 138.15 31.818309) (end 138.159745 31.808564) (width 5.1) (layer "B.Cu") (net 3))
 (segment (start 138.15 43.258325) (end 138.15 31.818309) (width 5.1) (layer "B.Cu") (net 3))
 (segment (start 139.42 28.952081) (end 139.42 27.75) (width 2.55) (layer "B.Cu") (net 3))
 (segment (start 143.231531 41.631531) (end 143.231531 32.978929) (width 5) (layer "F.Cu") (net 4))
 (segment (start 142.032977 30.290902) (end 142.429098 30.290902) (width 0.25) (layer "F.Cu") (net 4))
 (segment (start 144.527402 30.271715) (end 144.508215 30.290902) (width 0.25) (layer "F.Cu") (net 4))
 (segment (start 144.5 30.29) (end 141.96 30.29) (width 2.5) (layer "F.Cu") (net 4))
 (segment (start 147 45.4) (end 143.231531 41.631531) (width 5) (layer "F.Cu") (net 4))
 (segment (start 141.96 30.29) (end 141.96 27.75) (width 2.5) (layer "F.Cu") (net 4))
 (segment (start 147 47) (end 147 45.4) (width 5) (layer "F.Cu") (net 4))
 (segment (start 144.5 30.29) (end 144.5 32.624762) (width 2.5) (layer "F.Cu") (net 4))
 (segment (start 142.013789 30.271714) (end 141.898661 30.156586) (width 0.25) (layer "F.Cu") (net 4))
 (segment (start 141.96 30.29) (end 141.96 32.74) (width 2.5) (layer "F.Cu") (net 4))
 (segment (start 141.96 27.75) (end 144.5 30.29) (width 1) (layer "F.Cu") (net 4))
 (segment (start 142.032977 30.290902) (end 142.013789 30.271714) (width 0.25) (layer "F.Cu") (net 4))
 (segment (start 141.96 30.195939) (end 141.976613 30.212552) (width 0.25) (layer "B.Cu") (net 4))
 (segment (start 141.96 27.75) (end 142.063064 27.75) (width 0.25) (layer "B.Cu") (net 4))
 (segment (start 142.410472 30.302095) (end 142.037374 30.302095) (width 0.25) (layer "B.Cu") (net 4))
 (segment (start 142.063064 27.75) (end 142.069354 27.74371) (width 0.25) (layer "B.Cu") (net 4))
 (segment (start 142.037374 30.302095) (end 141.983009 30.24773) (width 0.25) (layer "B.Cu") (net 4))
 (segment (start 144.567084 30.257218) (end 144.54779 30.276512) (width 0.25) (layer "B.Cu") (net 4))
 (segment (start 134.34 27.75) (end 133.058423 29.031577) (width 0.25) (layer "F.Cu") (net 2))
 (segment (start 133.058423 49.808423) (end 134.75 51.5) (width 0.25) (layer "F.Cu") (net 2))
 (segment (start 133.058423 29.031577) (end 133.058423 49.808423) (width 0.25) (layer "F.Cu") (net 2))
 (segment (start 125.909979 24.399979) (end 120.158301 24.399979) (width 0.76) (layer "F.Cu") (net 8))
 (segment (start 121.267846 45) (end 124.75 45) (width 0.76) (layer "F.Cu") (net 8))
 (segment (start 129.26 27.75) (end 125.909979 24.399979) (width 0.76) (layer "F.Cu") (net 8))
 (segment (start 120.158301 24.399979) (end 115.821563 28.736717) (width 0.76) (layer "F.Cu") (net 8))
 (segment (start 115.821563 28.736717) (end 115.821563 39.553717) (width 0.76) (layer "F.Cu") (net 8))
 (segment (start 115.821563 39.553717) (end 121.267846 45) (width 0.76) (layer "F.Cu") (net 8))
 (segment (start 124.75 42.147339) (end 124.75 42.5) (width 0.76) (layer "F.Cu") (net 7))
 (segment (start 124.329989 25.359989) (end 120.55595 25.359989) (width 0.76) (layer "F.Cu") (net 7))
 (segment (start 120.55595 25.359989) (end 118.289979 27.62596) (width 0.76) (layer "F.Cu") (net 7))
 (segment (start 118.289979 35.687318) (end 124.75 42.147339) (width 0.76) (layer "F.Cu") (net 7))
 (segment (start 118.289979 27.62596) (end 118.289979 35.687318) (width 0.76) (layer "F.Cu") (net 7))
 (segment (start 126.72 27.75) (end 124.329989 25.359989) (width 0.76) (layer "F.Cu") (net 7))
 (segment (start 122.066291 48.611573) (end 122.066291 33.785704) (width 2.25) (layer "B.Cu") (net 13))
 (segment (start 124.18 30.29) (end 124.18 27.75) (width 2.25) (layer "B.Cu") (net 13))
 (segment (start 119.177864 51.5) (end 122.066291 48.611573) (width 2.25) (layer "B.Cu") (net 13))
 (segment (start 117.5 51.5) (end 119.177864 51.5) (width 2.25) (layer "B.Cu") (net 13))
 (segment (start 122.066291 33.785704) (end 124.18 31.671995) (width 2.25) (layer "B.Cu") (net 13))
 (segment (start 124.18 31.671995) (end 124.18 30.29) (width 2.25) (layer "B.Cu") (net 13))
 (segment (start 131.8 27.75) (end 131.8 43.507903) (width 2.5) (layer "B.Cu") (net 11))
 (segment (start 124.553441 54) (end 123.25 54) (width 2.5) (layer "B.Cu") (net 11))
 (segment (start 126.238525 49.069378) (end 126.238525 52.314916) (width 2.5) (layer "B.Cu") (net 11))
 (segment (start 126.238525 52.314916) (end 124.553441 54) (width 2.5) (layer "B.Cu") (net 11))
 (segment (start 131.8 43.507903) (end 126.238525 49.069378) (width 2.5) (layer "B.Cu") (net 11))
 (segment (start 123.25 54) (end 117.5 54) (width 2.25) (layer "B.Cu") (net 11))
 (segment (start 131.8 30.29) (end 131.89 30.29) (width 1.5) (layer "B.Cu") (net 11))
 (segment (start 129.26 45.49) (end 123.25 51.5) (width 1.27) (layer "F.Cu") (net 12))
 (segment (start 129.26 30.29) (end 129.26 45.49) (width 1.27) (layer "F.Cu") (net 12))
 (segment (start 120.209999 29.180001) (end 120.209999 32.959999) (width 0.76) (layer "F.Cu") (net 5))
 (segment (start 121.64 27.75) (end 120.209999 29.180001) (width 0.76) (layer "F.Cu") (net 5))
 (segment (start 120.209999 32.959999) (end 124.75 37.5) (width 0.76) (layer "F.Cu") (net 5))
 (segment (start 144.480926 27.75) (end 144.527402 27.796476) (width 0.25) (layer "F.Cu") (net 9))
 (segment (start 130.337738 55.337738) (end 129 54) (width 0.25) (layer "B.Cu") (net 9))
 (segment (start 144.96573 49.450736) (end 139.078728 55.337738) (width 0.25) (layer "B.Cu") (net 9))
 (segment (start 139.078728 55.337738) (end 130.337738 55.337738) (width 0.25) (layer "B.Cu") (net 9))
 (segment (start 144.567084 27.75) (end 144.630938 27.686146) (width 0.25) (layer "B.Cu") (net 9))
 (segment (start 144.5 27.75) (end 145.989343 29.239343) (width 0.25) (layer "B.Cu") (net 9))
 (segment (start 144.96573 33.15138) (end 144.96573 49.450736) (width 0.25) (layer "B.Cu") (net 9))
 (segment (start 144.5 27.75) (end 144.59 27.75) (width 0.25) (layer "B.Cu") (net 9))
 (segment (start 145.989343 29.239343) (end 145.989343 32.127767) (width 0.25) (layer "B.Cu") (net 9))
 (segment (start 145.989343 32.127767) (end 144.96573 33.15138) (width 0.25) (layer "B.Cu") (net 9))
 (segment (start 126.72 38.388742) (end 125.108742 40) (width 0.76) (layer "F.Cu") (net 6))
 (segment (start 126.72 30.29) (end 126.72 38.388742) (width 0.76) (layer "F.Cu") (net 6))
 (segment (start 125.108742 40) (end 124.75 40) (width 1.27) (layer "F.Cu") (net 6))
 (segment (start 135.523976 26.393976) (end 131.164692 26.393976) (width 0.25) (layer "F.Cu") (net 10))
 (segment (start 131.164692 26.393976) (end 130.434511 27.124157) (width 0.25) (layer "F.Cu") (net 10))
 (segment (start 130.434511 27.124157) (end 130.434511 50.065489) (width 0.25) (layer "F.Cu") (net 10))
 (segment (start 130.434511 50.065489) (end 129 51.5) (width 0.25) (layer "F.Cu") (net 10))
 (segment (start 136.88 27.75) (end 135.523976 26.393976) (width 0.25) (layer "F.Cu") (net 10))
 (segment (start 136.88 27.768721) (end 136.871433 27.777288) (width 0.5) (layer "B.Cu") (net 10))
 (segment (start 136.88 27.75) (end 136.88 27.768721) (width 0.5) (layer "B.Cu") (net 10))
 (segment (start 136.898721 27.75) (end 136.871433 27.777288) (width 0.25) (layer "B.Cu") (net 10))
 (segment (start 137.35 27.75) (end 137.16 27.94) (width 0.25) (layer "B.Cu") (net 10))
 (segment (start 136.871433 27.777288) (end 136.907288 27.777288) (width 0.25) (layer "B.Cu") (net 10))
 (segment (start 121.64 30.29) (end 120.237647 31.692353) (width 0.5) (layer "B.Cu") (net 14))
 (segment (start 120.237647 46.262353) (end 117.5 49) (width 0.5) (layer "B.Cu") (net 14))
 (segment (start 120.237647 31.692353) (end 120.237647 46.262353) (width 0.5) (layer "B.Cu") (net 14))
 (segment (start 134.34 30.29) (end 134.62 30.57) (width 0.25) (layer "F.Cu") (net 1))
 (segment (start 136.213926 50.872731) (end 136.213926 52.536074) (width 0.25) (layer "F.Cu") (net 1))
 (segment (start 134.62 30.57) (end 134.62 49.278805) (width 0.25) (layer "F.Cu") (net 1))
 (segment (start 134.62 49.278805) (end 136.213926 50.872731) (width 0.25) (layer "F.Cu") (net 1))
 (segment (start 136.213926 52.536074) (end 134.75 54) (width 0.25) (layer "F.Cu") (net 1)))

